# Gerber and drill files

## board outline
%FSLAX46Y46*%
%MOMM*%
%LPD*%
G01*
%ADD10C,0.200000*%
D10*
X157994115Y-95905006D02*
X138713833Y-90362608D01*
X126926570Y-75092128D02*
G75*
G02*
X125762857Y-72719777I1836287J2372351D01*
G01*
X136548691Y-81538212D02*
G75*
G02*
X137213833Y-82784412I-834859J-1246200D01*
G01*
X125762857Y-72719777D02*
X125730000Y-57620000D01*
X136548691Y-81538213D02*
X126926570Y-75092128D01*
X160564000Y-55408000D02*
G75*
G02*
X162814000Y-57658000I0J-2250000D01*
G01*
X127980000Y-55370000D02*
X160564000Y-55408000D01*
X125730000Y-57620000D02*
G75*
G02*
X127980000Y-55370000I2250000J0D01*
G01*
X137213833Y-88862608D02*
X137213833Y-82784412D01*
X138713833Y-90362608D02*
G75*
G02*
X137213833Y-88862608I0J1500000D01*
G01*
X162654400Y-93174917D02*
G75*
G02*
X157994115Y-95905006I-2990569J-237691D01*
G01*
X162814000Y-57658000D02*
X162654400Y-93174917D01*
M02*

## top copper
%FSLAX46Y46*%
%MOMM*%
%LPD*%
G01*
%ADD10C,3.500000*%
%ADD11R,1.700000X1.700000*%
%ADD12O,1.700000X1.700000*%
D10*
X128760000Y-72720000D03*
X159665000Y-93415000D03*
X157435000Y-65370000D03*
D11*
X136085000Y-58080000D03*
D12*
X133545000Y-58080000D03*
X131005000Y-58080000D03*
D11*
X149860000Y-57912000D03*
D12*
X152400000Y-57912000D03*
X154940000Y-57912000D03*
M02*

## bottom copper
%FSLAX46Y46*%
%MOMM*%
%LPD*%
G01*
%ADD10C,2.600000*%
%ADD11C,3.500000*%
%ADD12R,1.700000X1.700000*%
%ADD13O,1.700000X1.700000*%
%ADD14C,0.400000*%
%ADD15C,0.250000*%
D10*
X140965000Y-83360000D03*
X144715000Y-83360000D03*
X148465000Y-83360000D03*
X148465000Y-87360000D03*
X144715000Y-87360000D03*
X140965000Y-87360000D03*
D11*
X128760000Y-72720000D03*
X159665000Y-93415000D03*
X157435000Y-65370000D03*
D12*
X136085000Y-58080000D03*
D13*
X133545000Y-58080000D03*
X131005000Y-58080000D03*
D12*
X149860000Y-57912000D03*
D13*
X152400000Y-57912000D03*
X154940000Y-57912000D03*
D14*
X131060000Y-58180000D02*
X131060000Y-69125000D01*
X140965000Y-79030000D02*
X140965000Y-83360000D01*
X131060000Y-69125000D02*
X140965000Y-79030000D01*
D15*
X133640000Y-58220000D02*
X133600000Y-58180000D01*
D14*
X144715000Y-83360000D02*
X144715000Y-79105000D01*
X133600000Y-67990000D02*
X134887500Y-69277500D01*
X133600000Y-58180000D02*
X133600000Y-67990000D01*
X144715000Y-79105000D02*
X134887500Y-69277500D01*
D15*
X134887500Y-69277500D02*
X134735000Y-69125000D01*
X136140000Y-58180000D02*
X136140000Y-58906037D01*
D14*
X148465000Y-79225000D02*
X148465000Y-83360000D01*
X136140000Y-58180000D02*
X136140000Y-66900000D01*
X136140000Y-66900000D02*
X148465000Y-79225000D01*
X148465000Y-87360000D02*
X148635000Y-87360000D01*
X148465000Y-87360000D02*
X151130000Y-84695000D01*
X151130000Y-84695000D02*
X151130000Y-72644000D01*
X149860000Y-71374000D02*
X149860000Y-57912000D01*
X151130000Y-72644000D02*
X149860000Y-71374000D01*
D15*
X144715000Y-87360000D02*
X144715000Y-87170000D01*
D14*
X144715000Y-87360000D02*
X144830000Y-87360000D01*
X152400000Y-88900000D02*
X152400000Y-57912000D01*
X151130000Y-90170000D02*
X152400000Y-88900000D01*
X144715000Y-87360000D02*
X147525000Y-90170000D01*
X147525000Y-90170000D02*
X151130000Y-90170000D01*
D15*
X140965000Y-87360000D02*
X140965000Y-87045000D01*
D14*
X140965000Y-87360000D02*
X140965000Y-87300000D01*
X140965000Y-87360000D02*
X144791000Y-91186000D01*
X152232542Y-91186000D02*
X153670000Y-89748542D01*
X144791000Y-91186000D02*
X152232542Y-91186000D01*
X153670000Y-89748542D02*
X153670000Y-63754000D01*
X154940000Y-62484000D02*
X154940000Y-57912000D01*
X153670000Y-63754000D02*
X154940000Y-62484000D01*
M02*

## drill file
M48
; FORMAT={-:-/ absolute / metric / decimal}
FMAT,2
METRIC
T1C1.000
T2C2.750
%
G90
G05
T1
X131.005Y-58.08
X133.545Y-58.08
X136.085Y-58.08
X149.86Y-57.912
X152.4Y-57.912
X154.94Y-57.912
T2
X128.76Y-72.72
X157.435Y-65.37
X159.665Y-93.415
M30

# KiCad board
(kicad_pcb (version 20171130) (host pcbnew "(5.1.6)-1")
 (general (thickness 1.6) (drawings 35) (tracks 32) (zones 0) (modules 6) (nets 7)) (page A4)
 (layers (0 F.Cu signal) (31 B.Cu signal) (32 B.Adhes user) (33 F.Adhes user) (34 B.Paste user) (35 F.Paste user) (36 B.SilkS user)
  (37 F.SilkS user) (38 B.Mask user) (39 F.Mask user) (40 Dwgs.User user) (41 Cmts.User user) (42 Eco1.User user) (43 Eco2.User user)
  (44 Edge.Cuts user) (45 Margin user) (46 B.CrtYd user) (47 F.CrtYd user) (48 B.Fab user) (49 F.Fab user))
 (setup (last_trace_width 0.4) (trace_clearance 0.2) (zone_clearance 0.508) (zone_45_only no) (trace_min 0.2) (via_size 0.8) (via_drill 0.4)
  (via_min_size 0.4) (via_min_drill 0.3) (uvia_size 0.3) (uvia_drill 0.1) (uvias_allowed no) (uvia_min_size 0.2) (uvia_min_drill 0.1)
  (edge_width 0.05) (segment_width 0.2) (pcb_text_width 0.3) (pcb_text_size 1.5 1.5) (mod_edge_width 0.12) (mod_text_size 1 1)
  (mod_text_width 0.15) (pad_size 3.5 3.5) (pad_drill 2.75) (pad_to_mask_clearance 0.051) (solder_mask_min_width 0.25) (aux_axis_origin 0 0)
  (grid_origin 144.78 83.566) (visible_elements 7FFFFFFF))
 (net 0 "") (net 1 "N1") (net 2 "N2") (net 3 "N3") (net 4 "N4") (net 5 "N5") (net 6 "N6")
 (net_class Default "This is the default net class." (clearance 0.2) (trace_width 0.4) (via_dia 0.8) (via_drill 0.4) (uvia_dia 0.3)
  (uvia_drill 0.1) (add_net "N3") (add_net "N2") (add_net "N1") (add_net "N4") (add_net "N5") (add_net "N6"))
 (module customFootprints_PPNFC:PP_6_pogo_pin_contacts (layer B.Cu) (at 148.465 83.36 180)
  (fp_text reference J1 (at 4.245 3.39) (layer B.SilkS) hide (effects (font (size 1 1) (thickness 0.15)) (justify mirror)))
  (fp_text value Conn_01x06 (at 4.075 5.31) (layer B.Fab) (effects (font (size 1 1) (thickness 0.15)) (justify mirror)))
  (pad 3 smd circle (at 7.5 0 180) (size 2.6 2.6) (layers B.Cu B.Paste B.Mask) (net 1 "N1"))
  (pad 2 smd circle (at 3.75 0 180) (size 2.6 2.6) (layers B.Cu B.Paste B.Mask) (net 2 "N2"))
  (pad 1 smd circle (at 0 0 180) (size 2.6 2.6) (layers B.Cu B.Paste B.Mask) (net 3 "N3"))
  (pad 4 smd circle (at 0 -4 180) (size 2.6 2.6) (layers B.Cu B.Paste B.Mask) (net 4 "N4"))
  (pad 5 smd circle (at 3.75 -4 180) (size 2.6 2.6) (layers B.Cu B.Paste B.Mask) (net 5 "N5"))
  (pad 6 smd circle (at 7.5 -4 180) (size 2.6 2.6) (layers B.Cu B.Paste B.Mask) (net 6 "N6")))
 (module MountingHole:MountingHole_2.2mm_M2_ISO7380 (layer F.Cu) (at 128.76 72.72)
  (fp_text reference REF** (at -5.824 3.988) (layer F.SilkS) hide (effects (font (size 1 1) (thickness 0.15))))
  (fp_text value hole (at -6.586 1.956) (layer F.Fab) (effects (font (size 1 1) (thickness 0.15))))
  (pad "" np_thru_hole circle (at 0 0) (size 3.5 3.5) (drill 2.75) (layers *.Cu *.Mask)))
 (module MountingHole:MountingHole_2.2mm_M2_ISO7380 (layer F.Cu) (at 159.665 93.415)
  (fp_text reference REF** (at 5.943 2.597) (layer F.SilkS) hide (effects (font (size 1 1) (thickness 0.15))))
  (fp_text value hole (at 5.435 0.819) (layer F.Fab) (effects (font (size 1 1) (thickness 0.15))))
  (pad "" np_thru_hole circle (at 0 0) (size 3.5 3.5) (drill 2.75) (layers *.Cu *.Mask)))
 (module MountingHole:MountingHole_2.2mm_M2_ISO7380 (layer F.Cu) (at 157.435 65.37)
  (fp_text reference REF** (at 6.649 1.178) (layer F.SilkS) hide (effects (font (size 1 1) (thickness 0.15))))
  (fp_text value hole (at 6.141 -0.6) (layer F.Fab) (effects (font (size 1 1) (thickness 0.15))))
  (pad "" np_thru_hole circle (at 0 0) (size 3.5 3.5) (drill 2.75) (layers *.Cu *.Mask)))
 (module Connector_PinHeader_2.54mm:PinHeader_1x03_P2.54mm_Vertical (layer F.Cu) (at 136.085 58.08 270)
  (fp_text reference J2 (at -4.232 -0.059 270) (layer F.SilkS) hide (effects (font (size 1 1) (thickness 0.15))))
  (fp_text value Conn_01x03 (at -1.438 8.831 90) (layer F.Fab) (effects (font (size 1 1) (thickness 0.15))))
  (pad 1 thru_hole rect (at 0 0 270) (size 1.7 1.7) (drill 1) (layers *.Cu *.Mask) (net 3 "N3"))
  (pad 2 thru_hole oval (at 0 2.54 270) (size 1.7 1.7) (drill 1) (layers *.Cu *.Mask) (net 2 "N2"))
  (pad 3 thru_hole oval (at 0 5.08 270) (size 1.7 1.7) (drill 1) (layers *.Cu *.Mask) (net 1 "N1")))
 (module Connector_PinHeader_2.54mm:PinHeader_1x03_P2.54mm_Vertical (layer F.Cu) (at 149.86 57.912 90)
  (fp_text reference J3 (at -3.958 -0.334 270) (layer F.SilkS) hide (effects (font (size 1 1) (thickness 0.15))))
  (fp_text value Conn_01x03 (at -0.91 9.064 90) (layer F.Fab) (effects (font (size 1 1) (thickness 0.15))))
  (pad 1 thru_hole rect (at 0 0 90) (size 1.7 1.7) (drill 1) (layers *.Cu *.Mask) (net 4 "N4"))
  (pad 2 thru_hole oval (at 0 2.54 90) (size 1.7 1.7) (drill 1) (layers *.Cu *.Mask) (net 5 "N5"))
  (pad 3 thru_hole oval (at 0 5.08 90) (size 1.7 1.7) (drill 1) (layers *.Cu *.Mask) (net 6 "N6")))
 (gr_line (start 157.994115 95.905006) (end 138.713833 90.362608) (layer Edge.Cuts) (width 0.2))
 (gr_arc (start 128.762857 72.719777) (end 125.762857 72.719777) (angle -52.25880262) (layer Edge.Cuts) (width 0.2))
 (gr_arc (start 135.713832 82.784412) (end 137.213833 82.784412) (angle -56.18093969) (layer Edge.Cuts) (width 0.2))
 (gr_line (start 125.762857 72.719777) (end 125.73 57.62) (layer Edge.Cuts) (width 0.2))
 (gr_line (start 136.548691 81.538213) (end 126.92657 75.092128) (layer Edge.Cuts) (width 0.2))
 (gr_arc (start 160.564 57.658) (end 162.814 57.658) (angle -90) (layer Edge.Cuts) (width 0.2))
 (gr_line (start 127.98 55.37) (end 160.564 55.408) (layer Edge.Cuts) (width 0.2))
 (gr_arc (start 127.98 57.62) (end 127.98 55.37) (angle -90) (layer Edge.Cuts) (width 0.2))
 (gr_line (start 137.213833 88.862608) (end 137.213833 82.784412) (layer Edge.Cuts) (width 0.2))
 (gr_arc (start 138.713833 88.862608) (end 137.213833 88.862608) (angle -90) (layer Edge.Cuts) (width 0.2))
 (gr_arc (start 159.663831 93.412608) (end 157.994115 95.905006) (angle -128.3633848) (layer Edge.Cuts) (width 0.2))
 (gr_line (start 162.814 57.658) (end 162.6544 93.174917) (layer Edge.Cuts) (width 0.2))
 (segment (start 131.06 58.18) (end 131.06 69.125) (width 0.4) (layer B.Cu) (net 1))
 (segment (start 140.965 79.03) (end 140.965 83.36) (width 0.4) (layer B.Cu) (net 1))
 (segment (start 131.06 69.125) (end 140.965 79.03) (width 0.4) (layer B.Cu) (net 1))
 (segment (start 133.64 58.22) (end 133.6 58.18) (width 0.25) (layer B.Cu) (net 2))
 (segment (start 144.715 83.36) (end 144.715 79.105) (width 0.4) (layer B.Cu) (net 2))
 (segment (start 133.6 67.99) (end 134.8875 69.2775) (width 0.4) (layer B.Cu) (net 2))
 (segment (start 133.6 58.18) (end 133.6 67.99) (width 0.4) (layer B.Cu) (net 2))
 (segment (start 144.715 79.105) (end 134.8875 69.2775) (width 0.4) (layer B.Cu) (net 2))
 (segment (start 134.8875 69.2775) (end 134.735 69.125) (width 0.25) (layer B.Cu) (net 2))
 (segment (start 136.14 58.18) (end 136.14 58.906037) (width 0.25) (layer B.Cu) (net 3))
 (segment (start 148.465 79.225) (end 148.465 83.36) (width 0.4) (layer B.Cu) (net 3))
 (segment (start 136.14 58.18) (end 136.14 66.9) (width 0.4) (layer B.Cu) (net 3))
 (segment (start 136.14 66.9) (end 148.465 79.225) (width 0.4) (layer B.Cu) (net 3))
 (segment (start 148.465 87.36) (end 148.635 87.36) (width 0.4) (layer B.Cu) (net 4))
 (segment (start 148.465 87.36) (end 151.13 84.695) (width 0.4) (layer B.Cu) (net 4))
 (segment (start 151.13 84.695) (end 151.13 72.644) (width 0.4) (layer B.Cu) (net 4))
 (segment (start 149.86 71.374) (end 149.86 57.912) (width 0.4) (layer B.Cu) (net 4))
 (segment (start 151.13 72.644) (end 149.86 71.374) (width 0.4) (layer B.Cu) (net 4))
 (segment (start 144.715 87.36) (end 144.715 87.17) (width 0.25) (layer B.Cu) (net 5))
 (segment (start 144.715 87.36) (end 144.83 87.36) (width 0.4) (layer B.Cu) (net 5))
 (segment (start 152.4 88.9) (end 152.4 57.912) (width 0.4) (layer B.Cu) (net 5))
 (segment (start 151.13 90.17) (end 152.4 88.9) (width 0.4) (layer B.Cu) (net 5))
 (segment (start 144.715 87.36) (end 147.525 90.17) (width 0.4) (layer B.Cu) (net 5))
 (segment (start 147.525 90.17) (end 151.13 90.17) (width 0.4) (layer B.Cu) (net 5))
 (segment (start 140.965 87.36) (end 140.965 87.045) (width 0.25) (layer B.Cu) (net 6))
 (segment (start 140.965 87.36) (end 140.965 87.3) (width 0.4) (layer B.Cu) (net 6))
 (segment (start 140.965 87.36) (end 144.791 91.186) (width 0.4) (layer B.Cu) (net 6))
 (segment (start 152.232542 91.186) (end 153.67 89.748542) (width 0.4) (layer B.Cu) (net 6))
 (segment (start 144.791 91.186) (end 152.232542 91.186) (width 0.4) (layer B.Cu) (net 6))
 (segment (start 153.67 89.748542) (end 153.67 63.754) (width 0.4) (layer B.Cu) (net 6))
 (segment (start 154.94 62.484) (end 154.94 57.912) (width 0.4) (layer B.Cu) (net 6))
 (segment (start 153.67 63.754) (end 154.94 62.484) (width 0.4) (layer B.Cu) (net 6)))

